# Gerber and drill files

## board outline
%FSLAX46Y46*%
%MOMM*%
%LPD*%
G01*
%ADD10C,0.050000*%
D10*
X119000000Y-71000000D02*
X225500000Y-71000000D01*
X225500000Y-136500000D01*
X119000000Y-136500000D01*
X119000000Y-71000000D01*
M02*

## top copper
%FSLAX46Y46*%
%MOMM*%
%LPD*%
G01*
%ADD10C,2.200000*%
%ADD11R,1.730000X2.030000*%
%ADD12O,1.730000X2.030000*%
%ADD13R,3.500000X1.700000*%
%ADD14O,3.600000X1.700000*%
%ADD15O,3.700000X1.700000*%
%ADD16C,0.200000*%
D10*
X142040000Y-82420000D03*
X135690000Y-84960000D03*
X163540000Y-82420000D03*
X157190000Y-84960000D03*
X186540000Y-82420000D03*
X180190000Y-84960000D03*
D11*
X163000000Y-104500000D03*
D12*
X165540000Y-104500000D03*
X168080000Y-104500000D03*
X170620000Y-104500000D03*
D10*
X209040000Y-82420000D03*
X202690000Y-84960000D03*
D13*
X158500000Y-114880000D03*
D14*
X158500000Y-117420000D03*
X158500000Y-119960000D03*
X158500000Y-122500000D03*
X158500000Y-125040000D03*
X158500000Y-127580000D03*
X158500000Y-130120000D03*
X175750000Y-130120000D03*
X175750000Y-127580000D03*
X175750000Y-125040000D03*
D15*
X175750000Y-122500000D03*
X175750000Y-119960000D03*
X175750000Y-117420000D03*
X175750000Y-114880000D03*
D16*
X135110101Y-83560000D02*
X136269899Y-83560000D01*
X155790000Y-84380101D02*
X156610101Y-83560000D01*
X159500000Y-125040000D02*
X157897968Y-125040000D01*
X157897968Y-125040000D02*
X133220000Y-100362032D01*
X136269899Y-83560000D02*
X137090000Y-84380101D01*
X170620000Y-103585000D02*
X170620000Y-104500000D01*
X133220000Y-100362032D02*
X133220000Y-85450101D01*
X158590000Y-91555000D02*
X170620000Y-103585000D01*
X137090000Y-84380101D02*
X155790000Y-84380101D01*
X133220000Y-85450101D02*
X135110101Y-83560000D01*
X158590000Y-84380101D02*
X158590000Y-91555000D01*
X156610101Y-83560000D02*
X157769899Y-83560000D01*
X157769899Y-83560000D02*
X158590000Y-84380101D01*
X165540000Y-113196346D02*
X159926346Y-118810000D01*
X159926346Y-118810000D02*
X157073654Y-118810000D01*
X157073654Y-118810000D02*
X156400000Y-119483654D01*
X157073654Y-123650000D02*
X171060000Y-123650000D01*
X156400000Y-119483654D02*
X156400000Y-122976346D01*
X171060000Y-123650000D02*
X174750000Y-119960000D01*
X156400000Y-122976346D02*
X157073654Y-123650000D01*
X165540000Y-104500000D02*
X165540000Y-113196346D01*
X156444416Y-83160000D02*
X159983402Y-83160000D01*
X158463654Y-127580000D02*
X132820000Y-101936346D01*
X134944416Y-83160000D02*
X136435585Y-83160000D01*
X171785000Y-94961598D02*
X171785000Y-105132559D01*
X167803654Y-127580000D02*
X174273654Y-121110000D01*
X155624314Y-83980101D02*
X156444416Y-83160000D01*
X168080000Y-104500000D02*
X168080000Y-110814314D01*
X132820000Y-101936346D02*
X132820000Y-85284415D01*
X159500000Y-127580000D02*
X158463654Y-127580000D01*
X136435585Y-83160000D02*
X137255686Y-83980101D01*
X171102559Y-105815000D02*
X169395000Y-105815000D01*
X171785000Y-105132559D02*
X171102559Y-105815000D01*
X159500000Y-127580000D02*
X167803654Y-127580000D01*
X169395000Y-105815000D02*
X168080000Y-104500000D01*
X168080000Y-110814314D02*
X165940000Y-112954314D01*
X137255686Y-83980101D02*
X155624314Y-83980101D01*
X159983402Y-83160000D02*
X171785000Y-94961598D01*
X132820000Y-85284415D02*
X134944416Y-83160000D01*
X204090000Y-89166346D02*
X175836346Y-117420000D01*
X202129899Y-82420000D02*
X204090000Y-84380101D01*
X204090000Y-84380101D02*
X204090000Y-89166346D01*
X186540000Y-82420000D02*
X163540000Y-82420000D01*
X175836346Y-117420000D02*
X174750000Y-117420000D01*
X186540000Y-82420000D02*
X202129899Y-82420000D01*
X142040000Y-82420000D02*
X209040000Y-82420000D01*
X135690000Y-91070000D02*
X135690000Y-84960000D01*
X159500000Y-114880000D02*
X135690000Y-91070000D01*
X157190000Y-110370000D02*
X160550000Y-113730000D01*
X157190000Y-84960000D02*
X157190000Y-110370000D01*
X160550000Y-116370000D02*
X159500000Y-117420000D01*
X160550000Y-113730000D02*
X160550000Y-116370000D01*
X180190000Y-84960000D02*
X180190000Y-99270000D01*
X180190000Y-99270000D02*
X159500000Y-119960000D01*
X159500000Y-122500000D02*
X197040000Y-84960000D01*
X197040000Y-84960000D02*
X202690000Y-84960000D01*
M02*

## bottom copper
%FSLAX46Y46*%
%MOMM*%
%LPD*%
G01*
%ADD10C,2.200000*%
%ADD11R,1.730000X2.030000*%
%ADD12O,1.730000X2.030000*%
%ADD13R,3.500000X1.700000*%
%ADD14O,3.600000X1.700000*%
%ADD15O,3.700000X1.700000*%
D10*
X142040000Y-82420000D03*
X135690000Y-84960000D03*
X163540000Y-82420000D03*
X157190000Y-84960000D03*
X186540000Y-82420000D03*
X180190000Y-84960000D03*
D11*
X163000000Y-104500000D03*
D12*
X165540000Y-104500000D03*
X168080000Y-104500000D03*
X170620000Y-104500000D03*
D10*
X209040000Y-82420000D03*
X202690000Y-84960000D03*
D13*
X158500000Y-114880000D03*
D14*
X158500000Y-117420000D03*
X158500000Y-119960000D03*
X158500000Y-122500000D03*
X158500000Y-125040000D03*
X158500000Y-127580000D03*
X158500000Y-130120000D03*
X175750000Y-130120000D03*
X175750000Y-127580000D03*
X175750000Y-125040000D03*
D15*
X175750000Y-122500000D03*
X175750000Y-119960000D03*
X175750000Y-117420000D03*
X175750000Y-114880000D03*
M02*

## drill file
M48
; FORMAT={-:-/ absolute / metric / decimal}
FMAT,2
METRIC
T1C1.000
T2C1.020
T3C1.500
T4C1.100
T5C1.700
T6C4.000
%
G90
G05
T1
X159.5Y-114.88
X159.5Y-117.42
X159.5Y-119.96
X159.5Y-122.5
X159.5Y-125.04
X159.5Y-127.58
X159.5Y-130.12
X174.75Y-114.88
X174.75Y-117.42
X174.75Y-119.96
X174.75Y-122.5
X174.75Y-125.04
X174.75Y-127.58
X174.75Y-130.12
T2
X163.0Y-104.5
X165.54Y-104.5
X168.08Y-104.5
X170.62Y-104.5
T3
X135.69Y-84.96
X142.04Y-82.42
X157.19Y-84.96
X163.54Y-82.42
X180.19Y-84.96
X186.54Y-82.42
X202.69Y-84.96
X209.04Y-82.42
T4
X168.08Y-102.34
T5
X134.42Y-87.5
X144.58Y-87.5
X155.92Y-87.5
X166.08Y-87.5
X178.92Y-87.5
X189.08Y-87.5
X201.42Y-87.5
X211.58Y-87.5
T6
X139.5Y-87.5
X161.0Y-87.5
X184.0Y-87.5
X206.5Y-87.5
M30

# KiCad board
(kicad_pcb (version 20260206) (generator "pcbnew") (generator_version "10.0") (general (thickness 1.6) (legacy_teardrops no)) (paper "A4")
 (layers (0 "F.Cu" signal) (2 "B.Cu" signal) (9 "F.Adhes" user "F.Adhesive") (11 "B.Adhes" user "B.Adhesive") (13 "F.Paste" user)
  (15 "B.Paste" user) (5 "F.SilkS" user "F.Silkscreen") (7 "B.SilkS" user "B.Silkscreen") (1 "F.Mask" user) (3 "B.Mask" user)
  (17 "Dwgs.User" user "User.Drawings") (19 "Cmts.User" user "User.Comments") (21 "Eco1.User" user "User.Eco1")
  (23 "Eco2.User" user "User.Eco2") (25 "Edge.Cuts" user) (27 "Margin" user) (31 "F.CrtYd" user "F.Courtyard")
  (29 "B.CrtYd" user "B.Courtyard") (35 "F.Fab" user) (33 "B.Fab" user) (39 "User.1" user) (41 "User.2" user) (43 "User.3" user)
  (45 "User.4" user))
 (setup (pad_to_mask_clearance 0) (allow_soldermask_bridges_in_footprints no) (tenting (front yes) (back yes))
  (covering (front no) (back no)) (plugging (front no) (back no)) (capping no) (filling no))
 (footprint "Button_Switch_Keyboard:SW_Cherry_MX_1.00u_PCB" (layer "F.Cu") (at 142.04 82.42)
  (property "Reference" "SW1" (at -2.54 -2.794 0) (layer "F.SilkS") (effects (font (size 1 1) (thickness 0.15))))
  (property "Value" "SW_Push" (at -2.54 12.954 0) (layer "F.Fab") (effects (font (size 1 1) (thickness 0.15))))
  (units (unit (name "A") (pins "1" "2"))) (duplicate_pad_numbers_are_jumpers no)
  (pad "" np_thru_hole circle (at -7.62 5.08) (size 1.7 1.7) (drill 1.7) (layers "*.Cu" "*.Mask"))
  (pad "" np_thru_hole circle (at -2.54 5.08) (size 4 4) (drill 4) (layers "*.Cu" "*.Mask"))
  (pad "" np_thru_hole circle (at 2.54 5.08) (size 1.7 1.7) (drill 1.7) (layers "*.Cu" "*.Mask"))
  (pad "1" thru_hole circle (at 0 0) (size 2.2 2.2) (drill 1.5) (layers "*.Cu" "*.Mask") (remove_unused_layers no) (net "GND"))
  (pad "2" thru_hole circle (at -6.35 2.54) (size 2.2 2.2) (drill 1.5) (layers "*.Cu" "*.Mask") (remove_unused_layers no)
   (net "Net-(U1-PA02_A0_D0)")))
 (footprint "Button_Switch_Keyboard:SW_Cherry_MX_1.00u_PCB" (layer "F.Cu") (at 163.54 82.42)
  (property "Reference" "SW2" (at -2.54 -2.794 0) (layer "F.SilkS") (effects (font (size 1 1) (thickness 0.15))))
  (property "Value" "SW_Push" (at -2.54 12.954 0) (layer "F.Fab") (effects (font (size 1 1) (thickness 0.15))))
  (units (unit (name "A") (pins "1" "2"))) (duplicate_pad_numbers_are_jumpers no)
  (pad "" np_thru_hole circle (at -7.62 5.08) (size 1.7 1.7) (drill 1.7) (layers "*.Cu" "*.Mask"))
  (pad "" np_thru_hole circle (at -2.54 5.08) (size 4 4) (drill 4) (layers "*.Cu" "*.Mask"))
  (pad "" np_thru_hole circle (at 2.54 5.08) (size 1.7 1.7) (drill 1.7) (layers "*.Cu" "*.Mask"))
  (pad "1" thru_hole circle (at 0 0) (size 2.2 2.2) (drill 1.5) (layers "*.Cu" "*.Mask") (remove_unused_layers no) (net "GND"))
  (pad "2" thru_hole circle (at -6.35 2.54) (size 2.2 2.2) (drill 1.5) (layers "*.Cu" "*.Mask") (remove_unused_layers no)
   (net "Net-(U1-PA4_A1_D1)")))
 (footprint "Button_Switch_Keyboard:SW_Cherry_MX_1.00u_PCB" (layer "F.Cu") (at 186.54 82.42)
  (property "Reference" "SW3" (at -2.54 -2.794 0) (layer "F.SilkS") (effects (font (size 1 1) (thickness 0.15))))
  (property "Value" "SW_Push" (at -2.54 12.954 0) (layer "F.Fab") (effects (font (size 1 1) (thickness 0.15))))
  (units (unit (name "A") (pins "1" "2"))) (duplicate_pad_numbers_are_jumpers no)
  (pad "" np_thru_hole circle (at -7.62 5.08) (size 1.7 1.7) (drill 1.7) (layers "*.Cu" "*.Mask"))
  (pad "" np_thru_hole circle (at -2.54 5.08) (size 4 4) (drill 4) (layers "*.Cu" "*.Mask"))
  (pad "" np_thru_hole circle (at 2.54 5.08) (size 1.7 1.7) (drill 1.7) (layers "*.Cu" "*.Mask"))
  (pad "1" thru_hole circle (at 0 0) (size 2.2 2.2) (drill 1.5) (layers "*.Cu" "*.Mask") (remove_unused_layers no) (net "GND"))
  (pad "2" thru_hole circle (at -6.35 2.54) (size 2.2 2.2) (drill 1.5) (layers "*.Cu" "*.Mask") (remove_unused_layers no)
   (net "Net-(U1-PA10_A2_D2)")))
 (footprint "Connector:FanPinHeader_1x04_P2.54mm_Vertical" (layer "F.Cu") (at 163 104.5)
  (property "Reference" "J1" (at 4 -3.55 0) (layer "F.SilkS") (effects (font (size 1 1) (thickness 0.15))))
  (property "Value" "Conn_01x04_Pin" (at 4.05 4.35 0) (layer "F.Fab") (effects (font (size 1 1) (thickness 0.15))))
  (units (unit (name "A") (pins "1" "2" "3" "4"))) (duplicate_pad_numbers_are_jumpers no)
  (pad "" np_thru_hole circle (at 5.08 -2.16 90) (size 1.1 1.1) (drill 1.1) (layers "*.Cu" "*.Mask"))
  (pad "1" thru_hole rect (at 0 0 90) (size 2.03 1.73) (drill 1.02) (layers "*.Cu" "*.Mask") (remove_unused_layers no)
   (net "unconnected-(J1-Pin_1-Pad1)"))
  (pad "2" thru_hole oval (at 2.54 0 90) (size 2.03 1.73) (drill 1.02) (layers "*.Cu" "*.Mask") (remove_unused_layers no)
   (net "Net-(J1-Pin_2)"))
  (pad "3" thru_hole oval (at 5.08 0 90) (size 2.03 1.73) (drill 1.02) (layers "*.Cu" "*.Mask") (remove_unused_layers no)
   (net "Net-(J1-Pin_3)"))
  (pad "4" thru_hole oval (at 7.62 0 90) (size 2.03 1.73) (drill 1.02) (layers "*.Cu" "*.Mask") (remove_unused_layers no)
   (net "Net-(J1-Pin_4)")))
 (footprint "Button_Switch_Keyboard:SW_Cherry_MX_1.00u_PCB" (layer "F.Cu") (at 209.04 82.42)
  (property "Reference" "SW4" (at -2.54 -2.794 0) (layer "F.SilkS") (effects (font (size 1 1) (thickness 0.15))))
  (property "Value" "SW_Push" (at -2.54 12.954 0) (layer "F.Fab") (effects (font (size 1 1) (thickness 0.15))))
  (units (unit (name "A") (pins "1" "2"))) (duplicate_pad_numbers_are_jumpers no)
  (pad "" np_thru_hole circle (at -7.62 5.08) (size 1.7 1.7) (drill 1.7) (layers "*.Cu" "*.Mask"))
  (pad "" np_thru_hole circle (at -2.54 5.08) (size 4 4) (drill 4) (layers "*.Cu" "*.Mask"))
  (pad "" np_thru_hole circle (at 2.54 5.08) (size 1.7 1.7) (drill 1.7) (layers "*.Cu" "*.Mask"))
  (pad "1" thru_hole circle (at 0 0) (size 2.2 2.2) (drill 1.5) (layers "*.Cu" "*.Mask") (remove_unused_layers no) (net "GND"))
  (pad "2" thru_hole circle (at -6.35 2.54) (size 2.2 2.2) (drill 1.5) (layers "*.Cu" "*.Mask") (remove_unused_layers no)
   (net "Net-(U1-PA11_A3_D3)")))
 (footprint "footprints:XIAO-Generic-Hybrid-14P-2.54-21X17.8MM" (layer "F.Cu") (at 167.125 122.5)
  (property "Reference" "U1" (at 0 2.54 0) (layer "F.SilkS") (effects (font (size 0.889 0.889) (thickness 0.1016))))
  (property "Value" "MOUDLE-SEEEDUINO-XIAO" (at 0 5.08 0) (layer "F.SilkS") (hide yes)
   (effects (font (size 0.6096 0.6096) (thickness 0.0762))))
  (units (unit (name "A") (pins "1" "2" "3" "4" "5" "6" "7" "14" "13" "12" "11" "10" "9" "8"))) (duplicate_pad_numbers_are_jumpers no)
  (pad "1" thru_hole rect (at -7.625 -7.62) (size 3.5 1.7) (drill 1 (offset -1 0)) (layers "*.Cu" "*.Mask") (remove_unused_layers no)
   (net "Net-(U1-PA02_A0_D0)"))
  (pad "2" thru_hole oval (at -7.625 -5.08) (size 3.6 1.7) (drill 1 (offset -1 0)) (layers "*.Cu" "*.Mask") (remove_unused_layers no)
   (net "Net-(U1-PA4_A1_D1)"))
  (pad "3" thru_hole oval (at -7.625 -2.54) (size 3.6 1.7) (drill 1 (offset -1 0)) (layers "*.Cu" "*.Mask") (remove_unused_layers no)
   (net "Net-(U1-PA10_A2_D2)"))
  (pad "4" thru_hole oval (at -7.625 0) (size 3.6 1.7) (drill 1 (offset -1 0)) (layers "*.Cu" "*.Mask") (remove_unused_layers no)
   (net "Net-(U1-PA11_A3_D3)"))
  (pad "5" thru_hole oval (at -7.625 2.54) (size 3.6 1.7) (drill 1 (offset -1 0)) (layers "*.Cu" "*.Mask") (remove_unused_layers no)
   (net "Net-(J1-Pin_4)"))
  (pad "6" thru_hole oval (at -7.625 5.08 180) (size 3.6 1.7) (drill 1 (offset 1 0)) (layers "*.Cu" "*.Mask") (remove_unused_layers no)
   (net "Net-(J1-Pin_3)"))
  (pad "7" thru_hole oval (at -7.625 7.62) (size 3.6 1.7) (drill 1 (offset -1 0)) (layers "*.Cu" "*.Mask") (remove_unused_layers no)
   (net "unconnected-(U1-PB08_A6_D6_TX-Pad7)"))
  (pad "8" thru_hole oval (at 7.625 7.62) (size 3.6 1.7) (drill 1 (offset 1 0)) (layers "*.Cu" "*.Mask") (remove_unused_layers no)
   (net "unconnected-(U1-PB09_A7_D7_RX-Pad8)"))
  (pad "9" thru_hole oval (at 7.625 5.08) (size 3.6 1.7) (drill 1 (offset 1 0)) (layers "*.Cu" "*.Mask") (remove_unused_layers no)
   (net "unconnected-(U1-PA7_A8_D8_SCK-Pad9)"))
  (pad "10" thru_hole oval (at 7.625 2.54) (size 3.6 1.7) (drill 1 (offset 1 0)) (layers "*.Cu" "*.Mask") (remove_unused_layers no)
   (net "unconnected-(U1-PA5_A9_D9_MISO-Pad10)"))
  (pad "11" thru_hole oval (at 7.625 0) (size 3.7 1.7) (drill 1 (offset 1 0)) (layers "*.Cu" "*.Mask") (remove_unused_layers no)
   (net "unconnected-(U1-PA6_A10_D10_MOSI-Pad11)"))
  (pad "12" thru_hole oval (at 7.625 -2.54) (size 3.7 1.7) (drill 1 (offset 1 0)) (layers "*.Cu" "*.Mask") (remove_unused_layers no)
   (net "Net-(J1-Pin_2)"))
  (pad "13" thru_hole oval (at 7.625 -5.08) (size 3.7 1.7) (drill 1 (offset 1 0)) (layers "*.Cu" "*.Mask") (remove_unused_layers no)
   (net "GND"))
  (pad "14" thru_hole oval (at 7.625 -7.62) (size 3.7 1.7) (drill 1 (offset 1 0)) (layers "*.Cu" "*.Mask") (remove_unused_layers no)
   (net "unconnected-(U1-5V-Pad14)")))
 (gr_rect (start 119 71) (end 225.5 136.5) (stroke (width 0.05) (type default)) (fill no) (layer "Edge.Cuts"))
 (segment (start 135.110101 83.56) (end 136.269899 83.56) (width 0.2) (layer "F.Cu") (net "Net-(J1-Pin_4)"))
 (segment (start 155.79 84.380101) (end 156.610101 83.56) (width 0.2) (layer "F.Cu") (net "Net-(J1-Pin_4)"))
 (segment (start 159.5 125.04) (end 157.897968 125.04) (width 0.2) (layer "F.Cu") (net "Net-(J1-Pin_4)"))
 (segment (start 157.897968 125.04) (end 133.22 100.362032) (width 0.2) (layer "F.Cu") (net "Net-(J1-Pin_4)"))
 (segment (start 136.269899 83.56) (end 137.09 84.380101) (width 0.2) (layer "F.Cu") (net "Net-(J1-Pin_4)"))
 (segment (start 170.62 103.585) (end 170.62 104.5) (width 0.2) (layer "F.Cu") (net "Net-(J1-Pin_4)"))
 (segment (start 133.22 100.362032) (end 133.22 85.450101) (width 0.2) (layer "F.Cu") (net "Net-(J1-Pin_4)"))
 (segment (start 158.59 91.555) (end 170.62 103.585) (width 0.2) (layer "F.Cu") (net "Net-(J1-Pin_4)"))
 (segment (start 137.09 84.380101) (end 155.79 84.380101) (width 0.2) (layer "F.Cu") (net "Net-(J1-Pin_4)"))
 (segment (start 133.22 85.450101) (end 135.110101 83.56) (width 0.2) (layer "F.Cu") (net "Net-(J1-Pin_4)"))
 (segment (start 158.59 84.380101) (end 158.59 91.555) (width 0.2) (layer "F.Cu") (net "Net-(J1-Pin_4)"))
 (segment (start 156.610101 83.56) (end 157.769899 83.56) (width 0.2) (layer "F.Cu") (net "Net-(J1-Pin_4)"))
 (segment (start 157.769899 83.56) (end 158.59 84.380101) (width 0.2) (layer "F.Cu") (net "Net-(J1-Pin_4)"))
 (segment (start 165.54 113.196346) (end 159.926346 118.81) (width 0.2) (layer "F.Cu") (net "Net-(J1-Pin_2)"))
 (segment (start 159.926346 118.81) (end 157.073654 118.81) (width 0.2) (layer "F.Cu") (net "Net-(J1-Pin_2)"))
 (segment (start 157.073654 118.81) (end 156.4 119.483654) (width 0.2) (layer "F.Cu") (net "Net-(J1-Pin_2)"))
 (segment (start 157.073654 123.65) (end 171.06 123.65) (width 0.2) (layer "F.Cu") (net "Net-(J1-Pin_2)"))
 (segment (start 156.4 119.483654) (end 156.4 122.976346) (width 0.2) (layer "F.Cu") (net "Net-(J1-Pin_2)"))
 (segment (start 171.06 123.65) (end 174.75 119.96) (width 0.2) (layer "F.Cu") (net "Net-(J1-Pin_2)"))
 (segment (start 156.4 122.976346) (end 157.073654 123.65) (width 0.2) (layer "F.Cu") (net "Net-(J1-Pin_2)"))
 (segment (start 165.54 104.5) (end 165.54 113.196346) (width 0.2) (layer "F.Cu") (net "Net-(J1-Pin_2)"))
 (segment (start 156.444416 83.16) (end 159.983402 83.16) (width 0.2) (layer "F.Cu") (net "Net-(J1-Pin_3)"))
 (segment (start 158.463654 127.58) (end 132.82 101.936346) (width 0.2) (layer "F.Cu") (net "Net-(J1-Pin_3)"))
 (segment (start 134.944416 83.16) (end 136.435585 83.16) (width 0.2) (layer "F.Cu") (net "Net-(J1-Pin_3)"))
 (segment (start 171.785 94.961598) (end 171.785 105.132559) (width 0.2) (layer "F.Cu") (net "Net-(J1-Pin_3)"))
 (segment (start 167.803654 127.58) (end 174.273654 121.11) (width 0.2) (layer "F.Cu") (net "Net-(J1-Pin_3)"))
 (segment (start 155.624314 83.980101) (end 156.444416 83.16) (width 0.2) (layer "F.Cu") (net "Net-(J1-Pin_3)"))
 (segment (start 168.08 104.5) (end 168.08 110.814314) (width 0.2) (layer "F.Cu") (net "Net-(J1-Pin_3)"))
 (segment (start 132.82 101.936346) (end 132.82 85.284415) (width 0.2) (layer "F.Cu") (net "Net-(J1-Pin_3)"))
 (segment (start 159.5 127.58) (end 158.463654 127.58) (width 0.2) (layer "F.Cu") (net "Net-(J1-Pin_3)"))
 (segment (start 136.435585 83.16) (end 137.255686 83.980101) (width 0.2) (layer "F.Cu") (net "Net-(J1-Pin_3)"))
 (segment (start 171.102559 105.815) (end 169.395 105.815) (width 0.2) (layer "F.Cu") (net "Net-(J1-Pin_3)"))
 (segment (start 171.785 105.132559) (end 171.102559 105.815) (width 0.2) (layer "F.Cu") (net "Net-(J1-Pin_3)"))
 (segment (start 159.5 127.58) (end 167.803654 127.58) (width 0.2) (layer "F.Cu") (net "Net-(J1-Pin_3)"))
 (segment (start 169.395 105.815) (end 168.08 104.5) (width 0.2) (layer "F.Cu") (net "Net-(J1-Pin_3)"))
 (segment (start 168.08 110.814314) (end 165.94 112.954314) (width 0.2) (layer "F.Cu") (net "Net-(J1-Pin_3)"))
 (segment (start 137.255686 83.980101) (end 155.624314 83.980101) (width 0.2) (layer "F.Cu") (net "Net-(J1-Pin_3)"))
 (segment (start 159.983402 83.16) (end 171.785 94.961598) (width 0.2) (layer "F.Cu") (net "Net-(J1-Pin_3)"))
 (segment (start 132.82 85.284415) (end 134.944416 83.16) (width 0.2) (layer "F.Cu") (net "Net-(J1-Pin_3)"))
 (segment (start 204.09 89.166346) (end 175.836346 117.42) (width 0.2) (layer "F.Cu") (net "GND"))
 (segment (start 202.129899 82.42) (end 204.09 84.380101) (width 0.2) (layer "F.Cu") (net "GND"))
 (segment (start 204.09 84.380101) (end 204.09 89.166346) (width 0.2) (layer "F.Cu") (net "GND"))
 (segment (start 186.54 82.42) (end 163.54 82.42) (width 0.2) (layer "F.Cu") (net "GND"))
 (segment (start 175.836346 117.42) (end 174.75 117.42) (width 0.2) (layer "F.Cu") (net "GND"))
 (segment (start 186.54 82.42) (end 202.129899 82.42) (width 0.2) (layer "F.Cu") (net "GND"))
 (segment (start 142.04 82.42) (end 209.04 82.42) (width 0.2) (layer "F.Cu") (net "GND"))
 (segment (start 135.69 91.07) (end 135.69 84.96) (width 0.2) (layer "F.Cu") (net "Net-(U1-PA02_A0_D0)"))
 (segment (start 159.5 114.88) (end 135.69 91.07) (width 0.2) (layer "F.Cu") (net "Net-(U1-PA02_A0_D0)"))
 (segment (start 157.19 110.37) (end 160.55 113.73) (width 0.2) (layer "F.Cu") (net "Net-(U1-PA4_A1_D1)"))
 (segment (start 157.19 84.96) (end 157.19 110.37) (width 0.2) (layer "F.Cu") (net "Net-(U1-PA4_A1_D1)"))
 (segment (start 160.55 116.37) (end 159.5 117.42) (width 0.2) (layer "F.Cu") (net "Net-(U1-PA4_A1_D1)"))
 (segment (start 160.55 113.73) (end 160.55 116.37) (width 0.2) (layer "F.Cu") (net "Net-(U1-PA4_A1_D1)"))
 (segment (start 180.19 84.96) (end 180.19 99.27) (width 0.2) (layer "F.Cu") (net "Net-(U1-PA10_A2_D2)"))
 (segment (start 180.19 99.27) (end 159.5 119.96) (width 0.2) (layer "F.Cu") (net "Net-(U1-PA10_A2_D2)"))
 (segment (start 159.5 122.5) (end 197.04 84.96) (width 0.2) (layer "F.Cu") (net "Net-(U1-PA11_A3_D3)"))
 (segment (start 197.04 84.96) (end 202.69 84.96) (width 0.2) (layer "F.Cu") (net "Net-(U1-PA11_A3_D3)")))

